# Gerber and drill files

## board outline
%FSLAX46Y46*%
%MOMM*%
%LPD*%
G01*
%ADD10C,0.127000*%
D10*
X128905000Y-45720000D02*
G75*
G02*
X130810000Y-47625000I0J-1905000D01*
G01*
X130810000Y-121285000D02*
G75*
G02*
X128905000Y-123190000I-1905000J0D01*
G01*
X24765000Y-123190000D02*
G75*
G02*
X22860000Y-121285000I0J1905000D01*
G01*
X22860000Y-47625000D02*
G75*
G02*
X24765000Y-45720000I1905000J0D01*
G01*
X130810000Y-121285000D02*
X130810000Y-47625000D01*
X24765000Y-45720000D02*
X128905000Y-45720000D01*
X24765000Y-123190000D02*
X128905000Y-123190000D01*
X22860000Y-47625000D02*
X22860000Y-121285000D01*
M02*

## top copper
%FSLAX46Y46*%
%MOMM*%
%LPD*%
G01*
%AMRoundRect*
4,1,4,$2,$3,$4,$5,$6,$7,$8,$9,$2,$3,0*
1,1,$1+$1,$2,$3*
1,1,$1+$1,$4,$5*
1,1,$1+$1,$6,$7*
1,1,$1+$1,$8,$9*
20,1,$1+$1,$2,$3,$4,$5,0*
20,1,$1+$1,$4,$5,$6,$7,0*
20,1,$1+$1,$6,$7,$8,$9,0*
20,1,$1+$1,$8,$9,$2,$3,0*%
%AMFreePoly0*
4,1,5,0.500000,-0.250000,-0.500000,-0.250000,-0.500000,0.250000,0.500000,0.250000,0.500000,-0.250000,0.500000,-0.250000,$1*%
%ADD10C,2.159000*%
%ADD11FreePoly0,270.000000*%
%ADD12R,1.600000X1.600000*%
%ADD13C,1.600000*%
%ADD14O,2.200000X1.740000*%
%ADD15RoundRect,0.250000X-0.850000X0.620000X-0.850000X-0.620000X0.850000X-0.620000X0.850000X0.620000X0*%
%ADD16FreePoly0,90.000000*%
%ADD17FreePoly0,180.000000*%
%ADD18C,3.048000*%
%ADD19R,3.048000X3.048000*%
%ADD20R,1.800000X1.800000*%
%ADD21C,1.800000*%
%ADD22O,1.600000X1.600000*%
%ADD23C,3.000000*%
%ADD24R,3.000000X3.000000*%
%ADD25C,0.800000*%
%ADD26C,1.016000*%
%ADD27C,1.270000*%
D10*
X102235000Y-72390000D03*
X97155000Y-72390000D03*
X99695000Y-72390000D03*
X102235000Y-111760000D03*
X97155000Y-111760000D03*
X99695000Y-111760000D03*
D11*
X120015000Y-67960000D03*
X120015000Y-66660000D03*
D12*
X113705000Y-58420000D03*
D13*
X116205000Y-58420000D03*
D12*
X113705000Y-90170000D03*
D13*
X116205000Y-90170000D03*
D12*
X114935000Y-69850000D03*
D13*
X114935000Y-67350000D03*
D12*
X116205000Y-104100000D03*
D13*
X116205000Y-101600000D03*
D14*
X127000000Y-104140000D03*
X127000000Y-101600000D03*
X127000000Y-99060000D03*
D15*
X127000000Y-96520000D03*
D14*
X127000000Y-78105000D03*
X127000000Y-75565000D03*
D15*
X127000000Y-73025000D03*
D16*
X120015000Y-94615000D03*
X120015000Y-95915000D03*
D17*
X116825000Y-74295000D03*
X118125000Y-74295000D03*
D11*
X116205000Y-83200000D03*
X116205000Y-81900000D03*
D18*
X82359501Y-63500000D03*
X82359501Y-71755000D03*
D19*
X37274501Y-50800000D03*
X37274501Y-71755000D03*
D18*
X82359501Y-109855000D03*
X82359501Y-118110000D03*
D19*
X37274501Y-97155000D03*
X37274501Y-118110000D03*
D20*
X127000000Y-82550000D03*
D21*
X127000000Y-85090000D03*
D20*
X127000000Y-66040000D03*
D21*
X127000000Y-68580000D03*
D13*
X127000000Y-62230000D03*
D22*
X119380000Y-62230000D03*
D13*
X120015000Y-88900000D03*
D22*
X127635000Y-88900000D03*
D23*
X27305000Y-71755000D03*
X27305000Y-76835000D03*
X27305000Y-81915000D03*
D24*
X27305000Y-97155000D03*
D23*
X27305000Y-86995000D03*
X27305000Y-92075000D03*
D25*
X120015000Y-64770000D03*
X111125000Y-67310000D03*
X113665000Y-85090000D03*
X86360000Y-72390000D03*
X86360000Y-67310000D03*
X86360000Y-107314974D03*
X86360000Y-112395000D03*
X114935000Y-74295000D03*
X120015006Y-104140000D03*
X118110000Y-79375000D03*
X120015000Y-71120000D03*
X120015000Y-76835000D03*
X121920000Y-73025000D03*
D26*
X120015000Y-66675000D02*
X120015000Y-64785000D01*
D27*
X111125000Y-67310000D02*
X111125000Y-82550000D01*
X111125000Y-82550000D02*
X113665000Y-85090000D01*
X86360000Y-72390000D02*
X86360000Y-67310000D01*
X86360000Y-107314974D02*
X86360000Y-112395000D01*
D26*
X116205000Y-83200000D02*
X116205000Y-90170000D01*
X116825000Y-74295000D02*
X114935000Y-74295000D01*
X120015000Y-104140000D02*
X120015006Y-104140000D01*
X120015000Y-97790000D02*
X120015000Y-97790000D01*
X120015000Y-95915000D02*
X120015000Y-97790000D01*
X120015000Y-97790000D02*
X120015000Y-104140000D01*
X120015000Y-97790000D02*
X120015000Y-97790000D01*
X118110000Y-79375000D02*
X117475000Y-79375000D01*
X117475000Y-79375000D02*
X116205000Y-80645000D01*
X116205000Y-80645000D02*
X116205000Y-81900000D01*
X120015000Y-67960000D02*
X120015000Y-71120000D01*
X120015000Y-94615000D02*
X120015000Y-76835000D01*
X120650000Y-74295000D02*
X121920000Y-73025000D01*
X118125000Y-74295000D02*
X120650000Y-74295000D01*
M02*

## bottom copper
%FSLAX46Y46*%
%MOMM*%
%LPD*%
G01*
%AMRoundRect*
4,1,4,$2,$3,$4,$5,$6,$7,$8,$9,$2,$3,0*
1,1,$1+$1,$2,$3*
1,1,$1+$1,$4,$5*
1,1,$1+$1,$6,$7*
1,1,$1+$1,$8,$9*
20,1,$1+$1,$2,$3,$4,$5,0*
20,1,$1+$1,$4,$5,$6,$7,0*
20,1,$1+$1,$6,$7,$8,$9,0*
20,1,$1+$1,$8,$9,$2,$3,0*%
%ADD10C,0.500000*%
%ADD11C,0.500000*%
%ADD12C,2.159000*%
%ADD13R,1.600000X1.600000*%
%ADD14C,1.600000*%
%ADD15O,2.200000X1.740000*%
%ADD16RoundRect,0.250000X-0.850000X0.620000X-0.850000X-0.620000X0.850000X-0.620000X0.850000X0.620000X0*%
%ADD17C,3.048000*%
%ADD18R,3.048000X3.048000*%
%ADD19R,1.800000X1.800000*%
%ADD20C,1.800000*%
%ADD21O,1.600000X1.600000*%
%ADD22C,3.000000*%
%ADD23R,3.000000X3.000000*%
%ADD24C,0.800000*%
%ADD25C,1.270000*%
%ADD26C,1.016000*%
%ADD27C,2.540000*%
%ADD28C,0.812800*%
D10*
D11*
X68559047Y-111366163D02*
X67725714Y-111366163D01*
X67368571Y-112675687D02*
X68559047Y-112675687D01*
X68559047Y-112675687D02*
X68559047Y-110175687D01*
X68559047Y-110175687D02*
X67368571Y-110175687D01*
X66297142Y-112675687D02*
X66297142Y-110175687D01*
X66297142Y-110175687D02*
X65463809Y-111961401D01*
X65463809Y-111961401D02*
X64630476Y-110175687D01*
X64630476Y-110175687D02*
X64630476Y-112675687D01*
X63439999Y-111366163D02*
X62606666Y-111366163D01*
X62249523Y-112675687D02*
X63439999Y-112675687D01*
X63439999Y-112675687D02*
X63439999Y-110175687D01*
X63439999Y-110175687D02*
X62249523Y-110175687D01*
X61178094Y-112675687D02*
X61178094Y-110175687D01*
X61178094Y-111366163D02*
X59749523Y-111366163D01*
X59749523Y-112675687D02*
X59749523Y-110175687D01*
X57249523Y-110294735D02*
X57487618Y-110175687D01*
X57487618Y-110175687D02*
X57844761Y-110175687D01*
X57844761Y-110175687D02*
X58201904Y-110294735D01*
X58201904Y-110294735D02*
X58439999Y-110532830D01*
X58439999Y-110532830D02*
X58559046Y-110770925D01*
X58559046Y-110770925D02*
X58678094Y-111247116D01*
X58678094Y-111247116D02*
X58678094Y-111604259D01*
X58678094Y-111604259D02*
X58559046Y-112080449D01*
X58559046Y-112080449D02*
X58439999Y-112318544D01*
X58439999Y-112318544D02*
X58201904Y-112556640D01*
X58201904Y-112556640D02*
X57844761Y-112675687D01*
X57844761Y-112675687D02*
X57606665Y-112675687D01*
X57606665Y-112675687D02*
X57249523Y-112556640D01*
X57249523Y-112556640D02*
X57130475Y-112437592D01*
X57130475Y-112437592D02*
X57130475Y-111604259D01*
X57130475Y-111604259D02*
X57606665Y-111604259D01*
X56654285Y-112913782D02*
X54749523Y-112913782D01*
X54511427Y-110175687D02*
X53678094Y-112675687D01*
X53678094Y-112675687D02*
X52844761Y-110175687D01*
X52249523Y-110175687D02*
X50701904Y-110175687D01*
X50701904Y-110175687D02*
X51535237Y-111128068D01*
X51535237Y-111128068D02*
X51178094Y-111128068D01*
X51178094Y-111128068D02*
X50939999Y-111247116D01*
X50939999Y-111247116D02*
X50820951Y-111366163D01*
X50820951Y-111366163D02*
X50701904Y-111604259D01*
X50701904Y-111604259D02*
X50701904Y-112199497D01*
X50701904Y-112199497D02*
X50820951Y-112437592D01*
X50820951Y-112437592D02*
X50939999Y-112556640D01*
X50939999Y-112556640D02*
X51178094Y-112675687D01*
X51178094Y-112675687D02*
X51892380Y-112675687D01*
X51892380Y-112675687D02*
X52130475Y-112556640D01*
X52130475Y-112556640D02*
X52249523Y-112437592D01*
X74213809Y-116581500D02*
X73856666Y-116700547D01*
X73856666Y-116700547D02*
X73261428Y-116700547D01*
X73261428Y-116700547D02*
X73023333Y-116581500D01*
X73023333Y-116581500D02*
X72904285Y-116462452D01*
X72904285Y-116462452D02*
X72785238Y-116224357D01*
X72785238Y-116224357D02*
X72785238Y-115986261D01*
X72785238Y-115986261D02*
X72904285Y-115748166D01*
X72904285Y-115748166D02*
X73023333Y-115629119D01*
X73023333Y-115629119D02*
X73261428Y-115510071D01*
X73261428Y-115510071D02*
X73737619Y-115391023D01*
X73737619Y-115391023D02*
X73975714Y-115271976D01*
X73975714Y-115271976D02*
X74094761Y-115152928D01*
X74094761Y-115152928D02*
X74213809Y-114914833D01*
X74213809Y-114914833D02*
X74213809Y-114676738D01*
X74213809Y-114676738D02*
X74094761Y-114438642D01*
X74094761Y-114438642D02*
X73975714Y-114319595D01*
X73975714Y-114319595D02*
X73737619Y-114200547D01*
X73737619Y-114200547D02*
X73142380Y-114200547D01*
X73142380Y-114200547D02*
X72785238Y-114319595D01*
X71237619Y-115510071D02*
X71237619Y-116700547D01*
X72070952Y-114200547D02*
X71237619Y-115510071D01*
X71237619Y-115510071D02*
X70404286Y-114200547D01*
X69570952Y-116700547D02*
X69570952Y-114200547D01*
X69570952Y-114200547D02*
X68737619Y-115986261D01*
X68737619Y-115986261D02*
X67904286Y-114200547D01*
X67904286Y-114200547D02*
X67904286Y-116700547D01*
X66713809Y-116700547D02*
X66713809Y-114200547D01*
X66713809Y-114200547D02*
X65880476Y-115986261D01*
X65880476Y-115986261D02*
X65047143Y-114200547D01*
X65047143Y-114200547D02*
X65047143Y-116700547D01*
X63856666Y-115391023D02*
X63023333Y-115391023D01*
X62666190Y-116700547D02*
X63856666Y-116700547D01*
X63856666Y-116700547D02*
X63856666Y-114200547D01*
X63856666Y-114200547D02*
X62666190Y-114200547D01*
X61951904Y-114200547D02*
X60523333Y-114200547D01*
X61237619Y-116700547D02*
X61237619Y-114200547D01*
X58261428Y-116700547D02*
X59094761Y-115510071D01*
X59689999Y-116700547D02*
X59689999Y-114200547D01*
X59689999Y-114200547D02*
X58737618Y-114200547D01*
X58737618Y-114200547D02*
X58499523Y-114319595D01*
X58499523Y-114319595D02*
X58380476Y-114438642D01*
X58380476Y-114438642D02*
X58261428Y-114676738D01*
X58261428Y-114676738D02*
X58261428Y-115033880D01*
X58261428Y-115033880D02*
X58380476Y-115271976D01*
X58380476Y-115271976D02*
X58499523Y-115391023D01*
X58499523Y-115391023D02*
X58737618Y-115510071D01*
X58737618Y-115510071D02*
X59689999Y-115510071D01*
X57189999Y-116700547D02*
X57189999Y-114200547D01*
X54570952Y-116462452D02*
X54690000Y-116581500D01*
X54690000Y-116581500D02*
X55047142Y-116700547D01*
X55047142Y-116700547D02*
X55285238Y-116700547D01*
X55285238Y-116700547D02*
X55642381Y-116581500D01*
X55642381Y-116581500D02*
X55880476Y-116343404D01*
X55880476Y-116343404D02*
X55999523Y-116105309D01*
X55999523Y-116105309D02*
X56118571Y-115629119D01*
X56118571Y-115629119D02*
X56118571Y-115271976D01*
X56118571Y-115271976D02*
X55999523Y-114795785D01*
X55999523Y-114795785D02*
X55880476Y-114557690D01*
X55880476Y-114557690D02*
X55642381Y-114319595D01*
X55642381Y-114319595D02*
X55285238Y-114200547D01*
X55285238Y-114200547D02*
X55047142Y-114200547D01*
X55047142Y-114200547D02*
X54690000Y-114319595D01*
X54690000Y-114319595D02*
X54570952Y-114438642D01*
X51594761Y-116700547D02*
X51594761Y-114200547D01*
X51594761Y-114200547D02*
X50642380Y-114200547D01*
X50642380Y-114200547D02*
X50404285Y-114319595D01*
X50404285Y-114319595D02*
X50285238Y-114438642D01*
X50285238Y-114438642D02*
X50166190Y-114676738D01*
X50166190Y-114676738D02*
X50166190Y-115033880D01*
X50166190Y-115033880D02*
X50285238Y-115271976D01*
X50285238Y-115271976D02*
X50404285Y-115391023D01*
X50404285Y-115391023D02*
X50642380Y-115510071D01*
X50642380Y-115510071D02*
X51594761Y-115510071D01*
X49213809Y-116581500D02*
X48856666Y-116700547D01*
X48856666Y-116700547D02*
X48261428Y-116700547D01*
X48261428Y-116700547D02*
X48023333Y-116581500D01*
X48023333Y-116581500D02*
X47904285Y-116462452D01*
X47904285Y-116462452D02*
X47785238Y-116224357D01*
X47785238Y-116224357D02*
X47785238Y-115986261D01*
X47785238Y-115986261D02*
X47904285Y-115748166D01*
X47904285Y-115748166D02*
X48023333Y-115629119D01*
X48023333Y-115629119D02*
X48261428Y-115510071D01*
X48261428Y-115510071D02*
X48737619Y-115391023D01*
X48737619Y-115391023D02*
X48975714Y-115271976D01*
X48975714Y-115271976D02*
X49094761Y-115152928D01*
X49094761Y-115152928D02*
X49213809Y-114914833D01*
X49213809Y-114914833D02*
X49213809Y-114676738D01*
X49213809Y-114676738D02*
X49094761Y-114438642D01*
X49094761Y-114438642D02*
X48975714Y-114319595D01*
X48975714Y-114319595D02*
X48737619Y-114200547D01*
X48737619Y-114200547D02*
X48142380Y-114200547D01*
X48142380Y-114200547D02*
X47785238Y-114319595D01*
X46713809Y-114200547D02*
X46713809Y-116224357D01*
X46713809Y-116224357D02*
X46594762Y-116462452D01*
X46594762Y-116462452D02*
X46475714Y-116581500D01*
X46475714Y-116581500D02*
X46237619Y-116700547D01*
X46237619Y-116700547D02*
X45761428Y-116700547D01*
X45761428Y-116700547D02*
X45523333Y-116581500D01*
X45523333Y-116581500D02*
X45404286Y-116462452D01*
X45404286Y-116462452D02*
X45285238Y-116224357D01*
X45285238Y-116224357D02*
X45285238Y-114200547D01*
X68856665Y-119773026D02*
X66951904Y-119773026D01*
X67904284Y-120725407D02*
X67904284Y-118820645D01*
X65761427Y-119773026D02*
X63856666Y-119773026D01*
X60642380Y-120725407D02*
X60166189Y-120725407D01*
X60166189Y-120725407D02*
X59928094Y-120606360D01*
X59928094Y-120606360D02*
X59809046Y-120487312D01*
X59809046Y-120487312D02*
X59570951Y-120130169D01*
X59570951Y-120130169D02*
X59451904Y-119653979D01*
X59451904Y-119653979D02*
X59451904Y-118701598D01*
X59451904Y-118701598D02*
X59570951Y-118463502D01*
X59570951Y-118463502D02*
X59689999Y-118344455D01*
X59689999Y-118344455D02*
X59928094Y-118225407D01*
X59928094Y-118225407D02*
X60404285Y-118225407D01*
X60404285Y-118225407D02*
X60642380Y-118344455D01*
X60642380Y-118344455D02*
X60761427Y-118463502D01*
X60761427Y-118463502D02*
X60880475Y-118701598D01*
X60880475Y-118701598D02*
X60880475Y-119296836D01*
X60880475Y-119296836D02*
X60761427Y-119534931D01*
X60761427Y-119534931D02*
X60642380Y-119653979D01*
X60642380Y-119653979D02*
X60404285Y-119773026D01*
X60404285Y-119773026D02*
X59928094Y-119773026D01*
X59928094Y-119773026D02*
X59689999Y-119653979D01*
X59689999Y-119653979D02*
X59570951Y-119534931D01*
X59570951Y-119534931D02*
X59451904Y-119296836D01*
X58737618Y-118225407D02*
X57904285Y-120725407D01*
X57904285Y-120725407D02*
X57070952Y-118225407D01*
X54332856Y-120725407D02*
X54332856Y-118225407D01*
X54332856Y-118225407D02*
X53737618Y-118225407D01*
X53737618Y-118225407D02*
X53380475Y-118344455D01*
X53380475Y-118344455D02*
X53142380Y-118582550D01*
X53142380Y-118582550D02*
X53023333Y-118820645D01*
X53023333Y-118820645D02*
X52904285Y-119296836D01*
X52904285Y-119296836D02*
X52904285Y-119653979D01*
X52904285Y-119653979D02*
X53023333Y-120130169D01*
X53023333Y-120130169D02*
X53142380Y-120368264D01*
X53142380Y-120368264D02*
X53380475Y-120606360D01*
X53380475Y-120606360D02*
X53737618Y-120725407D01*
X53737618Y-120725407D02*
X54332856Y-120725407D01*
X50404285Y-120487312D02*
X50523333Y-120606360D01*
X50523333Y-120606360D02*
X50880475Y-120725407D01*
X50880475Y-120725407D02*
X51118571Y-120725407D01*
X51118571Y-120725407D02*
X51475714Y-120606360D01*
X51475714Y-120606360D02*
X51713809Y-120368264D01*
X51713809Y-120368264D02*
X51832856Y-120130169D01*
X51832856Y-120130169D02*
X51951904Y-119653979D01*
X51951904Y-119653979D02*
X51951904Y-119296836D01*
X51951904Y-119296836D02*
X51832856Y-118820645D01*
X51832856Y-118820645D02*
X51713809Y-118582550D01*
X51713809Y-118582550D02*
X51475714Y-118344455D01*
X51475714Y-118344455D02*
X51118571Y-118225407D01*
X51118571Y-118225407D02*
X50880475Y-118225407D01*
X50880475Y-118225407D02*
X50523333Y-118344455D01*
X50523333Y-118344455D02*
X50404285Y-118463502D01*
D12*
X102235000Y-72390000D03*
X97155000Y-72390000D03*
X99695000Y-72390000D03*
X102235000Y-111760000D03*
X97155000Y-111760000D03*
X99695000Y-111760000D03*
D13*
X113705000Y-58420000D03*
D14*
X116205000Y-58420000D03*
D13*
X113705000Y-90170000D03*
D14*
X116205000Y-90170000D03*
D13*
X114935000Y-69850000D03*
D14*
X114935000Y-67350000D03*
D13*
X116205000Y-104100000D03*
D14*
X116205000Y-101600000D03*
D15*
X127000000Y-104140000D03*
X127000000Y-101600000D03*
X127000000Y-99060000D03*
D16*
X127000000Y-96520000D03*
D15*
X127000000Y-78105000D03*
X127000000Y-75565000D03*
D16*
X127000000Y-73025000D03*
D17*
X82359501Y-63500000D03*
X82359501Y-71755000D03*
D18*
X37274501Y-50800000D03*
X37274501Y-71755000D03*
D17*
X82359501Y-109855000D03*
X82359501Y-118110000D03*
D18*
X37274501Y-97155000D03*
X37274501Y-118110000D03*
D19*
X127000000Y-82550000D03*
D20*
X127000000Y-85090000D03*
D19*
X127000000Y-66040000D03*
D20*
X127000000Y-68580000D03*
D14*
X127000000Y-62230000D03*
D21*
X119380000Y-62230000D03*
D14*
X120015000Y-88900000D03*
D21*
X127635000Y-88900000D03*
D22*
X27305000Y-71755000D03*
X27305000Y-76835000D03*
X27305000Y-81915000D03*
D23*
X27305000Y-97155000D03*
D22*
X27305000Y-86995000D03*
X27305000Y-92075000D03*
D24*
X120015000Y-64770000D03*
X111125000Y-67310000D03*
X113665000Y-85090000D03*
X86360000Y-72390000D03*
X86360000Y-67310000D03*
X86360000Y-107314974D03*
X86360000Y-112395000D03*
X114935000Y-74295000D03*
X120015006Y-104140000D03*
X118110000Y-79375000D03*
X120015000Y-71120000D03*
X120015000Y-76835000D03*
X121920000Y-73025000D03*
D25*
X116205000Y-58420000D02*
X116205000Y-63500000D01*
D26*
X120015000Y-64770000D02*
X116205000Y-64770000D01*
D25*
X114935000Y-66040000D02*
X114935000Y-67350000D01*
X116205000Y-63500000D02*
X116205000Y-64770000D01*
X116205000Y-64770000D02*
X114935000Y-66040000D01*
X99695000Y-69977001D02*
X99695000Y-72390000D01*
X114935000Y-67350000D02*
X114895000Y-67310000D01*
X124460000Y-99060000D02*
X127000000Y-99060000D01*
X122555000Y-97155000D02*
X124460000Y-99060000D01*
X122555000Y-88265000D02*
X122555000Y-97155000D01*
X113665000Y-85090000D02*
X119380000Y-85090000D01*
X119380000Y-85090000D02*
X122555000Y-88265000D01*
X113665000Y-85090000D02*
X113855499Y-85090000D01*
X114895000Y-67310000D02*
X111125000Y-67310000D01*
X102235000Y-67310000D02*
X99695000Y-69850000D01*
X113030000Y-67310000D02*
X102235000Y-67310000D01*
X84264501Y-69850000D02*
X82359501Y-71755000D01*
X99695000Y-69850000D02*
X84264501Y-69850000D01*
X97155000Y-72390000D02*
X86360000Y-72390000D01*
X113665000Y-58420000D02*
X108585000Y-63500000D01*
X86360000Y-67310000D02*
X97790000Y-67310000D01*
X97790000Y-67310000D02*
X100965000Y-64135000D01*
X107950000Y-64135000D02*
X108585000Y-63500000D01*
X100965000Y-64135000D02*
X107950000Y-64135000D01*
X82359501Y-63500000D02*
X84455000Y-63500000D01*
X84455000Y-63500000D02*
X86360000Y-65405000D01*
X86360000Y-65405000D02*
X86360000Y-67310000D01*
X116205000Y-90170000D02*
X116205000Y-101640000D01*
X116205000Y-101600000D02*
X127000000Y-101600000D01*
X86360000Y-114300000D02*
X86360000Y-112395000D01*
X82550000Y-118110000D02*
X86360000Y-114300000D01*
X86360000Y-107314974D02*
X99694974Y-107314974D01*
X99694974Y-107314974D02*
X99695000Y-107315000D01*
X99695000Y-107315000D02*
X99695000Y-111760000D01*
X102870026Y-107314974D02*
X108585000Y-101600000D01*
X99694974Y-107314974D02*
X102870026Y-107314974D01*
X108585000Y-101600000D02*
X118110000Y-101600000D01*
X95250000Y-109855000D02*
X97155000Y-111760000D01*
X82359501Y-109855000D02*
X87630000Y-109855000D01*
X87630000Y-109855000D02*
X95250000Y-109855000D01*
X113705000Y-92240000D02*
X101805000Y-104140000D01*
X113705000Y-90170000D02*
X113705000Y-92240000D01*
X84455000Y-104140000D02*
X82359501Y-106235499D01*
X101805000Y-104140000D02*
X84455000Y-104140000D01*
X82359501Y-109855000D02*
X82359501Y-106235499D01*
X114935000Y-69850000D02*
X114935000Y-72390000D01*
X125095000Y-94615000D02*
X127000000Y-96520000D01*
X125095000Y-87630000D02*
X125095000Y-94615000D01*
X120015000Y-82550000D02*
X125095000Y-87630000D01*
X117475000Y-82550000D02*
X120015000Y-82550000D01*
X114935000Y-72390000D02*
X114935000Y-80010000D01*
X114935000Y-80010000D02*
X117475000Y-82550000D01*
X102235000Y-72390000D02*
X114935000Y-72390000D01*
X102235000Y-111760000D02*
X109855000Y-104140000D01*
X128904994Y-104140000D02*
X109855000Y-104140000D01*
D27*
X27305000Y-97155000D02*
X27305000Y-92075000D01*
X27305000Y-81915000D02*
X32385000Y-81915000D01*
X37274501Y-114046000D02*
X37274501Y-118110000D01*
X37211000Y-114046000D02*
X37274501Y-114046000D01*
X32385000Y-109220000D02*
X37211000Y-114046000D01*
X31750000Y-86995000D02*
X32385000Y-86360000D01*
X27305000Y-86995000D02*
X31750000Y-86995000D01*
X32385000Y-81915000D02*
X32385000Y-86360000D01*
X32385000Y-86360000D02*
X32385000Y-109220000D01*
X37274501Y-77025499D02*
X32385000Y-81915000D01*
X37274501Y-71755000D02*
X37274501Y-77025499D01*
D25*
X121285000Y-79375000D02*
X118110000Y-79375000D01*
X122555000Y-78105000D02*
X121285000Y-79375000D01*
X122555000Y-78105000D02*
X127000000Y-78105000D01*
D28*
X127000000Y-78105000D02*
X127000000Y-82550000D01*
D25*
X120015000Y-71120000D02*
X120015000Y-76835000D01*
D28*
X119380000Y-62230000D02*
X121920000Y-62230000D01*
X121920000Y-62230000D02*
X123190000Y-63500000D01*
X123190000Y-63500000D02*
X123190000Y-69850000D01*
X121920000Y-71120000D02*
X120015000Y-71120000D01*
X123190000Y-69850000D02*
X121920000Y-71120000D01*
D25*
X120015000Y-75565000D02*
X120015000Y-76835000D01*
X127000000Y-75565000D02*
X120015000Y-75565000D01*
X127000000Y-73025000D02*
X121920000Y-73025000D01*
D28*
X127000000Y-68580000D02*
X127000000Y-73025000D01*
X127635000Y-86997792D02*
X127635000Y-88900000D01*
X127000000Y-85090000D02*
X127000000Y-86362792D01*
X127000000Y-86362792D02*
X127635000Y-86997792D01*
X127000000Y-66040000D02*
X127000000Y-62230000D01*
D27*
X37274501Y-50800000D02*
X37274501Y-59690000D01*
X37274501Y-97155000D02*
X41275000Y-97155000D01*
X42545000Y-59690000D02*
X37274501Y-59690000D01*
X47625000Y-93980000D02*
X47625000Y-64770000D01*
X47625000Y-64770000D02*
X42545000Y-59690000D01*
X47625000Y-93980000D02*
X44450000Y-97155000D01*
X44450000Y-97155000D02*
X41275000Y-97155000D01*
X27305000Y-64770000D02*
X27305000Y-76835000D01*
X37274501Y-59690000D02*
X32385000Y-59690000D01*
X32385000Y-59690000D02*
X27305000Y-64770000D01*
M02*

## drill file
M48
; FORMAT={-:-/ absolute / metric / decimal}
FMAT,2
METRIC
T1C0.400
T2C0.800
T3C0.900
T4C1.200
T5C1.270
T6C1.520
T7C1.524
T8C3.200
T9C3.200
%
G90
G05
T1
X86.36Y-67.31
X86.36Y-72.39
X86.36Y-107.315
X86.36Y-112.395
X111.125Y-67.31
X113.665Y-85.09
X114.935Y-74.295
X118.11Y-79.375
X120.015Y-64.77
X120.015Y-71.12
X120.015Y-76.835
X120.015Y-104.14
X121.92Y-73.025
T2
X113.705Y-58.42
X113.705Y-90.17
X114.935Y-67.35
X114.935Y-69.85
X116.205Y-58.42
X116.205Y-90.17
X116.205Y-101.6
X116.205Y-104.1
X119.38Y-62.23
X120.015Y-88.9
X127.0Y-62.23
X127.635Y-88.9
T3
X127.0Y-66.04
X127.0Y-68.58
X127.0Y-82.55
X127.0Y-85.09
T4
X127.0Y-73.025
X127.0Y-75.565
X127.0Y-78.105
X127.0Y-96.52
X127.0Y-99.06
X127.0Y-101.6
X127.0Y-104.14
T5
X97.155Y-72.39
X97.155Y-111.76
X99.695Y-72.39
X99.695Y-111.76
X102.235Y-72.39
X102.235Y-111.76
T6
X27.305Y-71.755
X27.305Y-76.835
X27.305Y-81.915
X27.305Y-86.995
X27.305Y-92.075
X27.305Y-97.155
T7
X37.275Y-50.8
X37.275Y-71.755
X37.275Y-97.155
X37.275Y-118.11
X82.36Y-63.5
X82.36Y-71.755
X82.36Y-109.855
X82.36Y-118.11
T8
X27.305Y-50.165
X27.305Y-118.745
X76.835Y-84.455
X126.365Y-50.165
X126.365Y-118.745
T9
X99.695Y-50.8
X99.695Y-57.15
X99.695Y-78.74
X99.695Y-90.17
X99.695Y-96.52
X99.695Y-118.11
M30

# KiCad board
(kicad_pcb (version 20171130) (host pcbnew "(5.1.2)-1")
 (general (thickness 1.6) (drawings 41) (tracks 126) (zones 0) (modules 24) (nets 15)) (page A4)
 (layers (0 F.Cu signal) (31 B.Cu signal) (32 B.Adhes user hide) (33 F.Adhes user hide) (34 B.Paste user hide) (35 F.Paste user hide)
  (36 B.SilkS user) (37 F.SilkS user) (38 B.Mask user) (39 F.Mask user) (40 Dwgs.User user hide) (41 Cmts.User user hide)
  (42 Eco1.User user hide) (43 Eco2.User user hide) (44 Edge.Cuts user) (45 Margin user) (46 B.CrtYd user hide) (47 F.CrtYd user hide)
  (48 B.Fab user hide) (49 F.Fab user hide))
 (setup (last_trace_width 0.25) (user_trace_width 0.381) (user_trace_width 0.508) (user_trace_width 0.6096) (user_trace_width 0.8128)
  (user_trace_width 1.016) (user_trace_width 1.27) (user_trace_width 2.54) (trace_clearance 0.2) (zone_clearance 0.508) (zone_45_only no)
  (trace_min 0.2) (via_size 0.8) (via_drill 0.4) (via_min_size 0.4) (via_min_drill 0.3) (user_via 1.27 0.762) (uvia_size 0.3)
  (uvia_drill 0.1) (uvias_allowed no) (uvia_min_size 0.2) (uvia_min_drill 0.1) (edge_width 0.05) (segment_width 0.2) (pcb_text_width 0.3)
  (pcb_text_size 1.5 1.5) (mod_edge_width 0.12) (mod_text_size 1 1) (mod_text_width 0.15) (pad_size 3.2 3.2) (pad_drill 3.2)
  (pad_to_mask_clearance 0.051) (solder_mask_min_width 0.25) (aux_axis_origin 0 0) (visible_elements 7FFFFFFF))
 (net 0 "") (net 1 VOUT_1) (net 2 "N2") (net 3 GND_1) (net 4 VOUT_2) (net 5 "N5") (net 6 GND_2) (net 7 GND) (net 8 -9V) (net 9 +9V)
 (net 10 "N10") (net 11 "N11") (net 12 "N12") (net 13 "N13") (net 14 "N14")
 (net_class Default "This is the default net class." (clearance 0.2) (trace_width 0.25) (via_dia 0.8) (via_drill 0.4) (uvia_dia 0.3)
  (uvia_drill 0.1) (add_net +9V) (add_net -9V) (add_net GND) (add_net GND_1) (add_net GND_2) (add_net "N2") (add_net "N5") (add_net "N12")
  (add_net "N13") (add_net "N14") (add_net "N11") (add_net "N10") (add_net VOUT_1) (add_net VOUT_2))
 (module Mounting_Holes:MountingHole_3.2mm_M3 (layer F.Cu) (at 76.835 84.455)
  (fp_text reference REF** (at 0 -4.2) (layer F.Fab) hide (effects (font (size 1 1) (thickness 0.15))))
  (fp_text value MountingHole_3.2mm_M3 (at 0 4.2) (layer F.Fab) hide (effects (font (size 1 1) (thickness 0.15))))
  (pad "" np_thru_hole circle (at 0 0) (size 3.2 3.2) (drill 3.2) (layers *.Cu *.Mask)))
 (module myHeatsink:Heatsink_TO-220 (layer F.Cu) (at 111.125 82.55 90)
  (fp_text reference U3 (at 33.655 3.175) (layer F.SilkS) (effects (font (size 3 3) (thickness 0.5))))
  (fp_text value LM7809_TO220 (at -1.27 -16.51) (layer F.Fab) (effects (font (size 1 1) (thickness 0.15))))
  (pad "" np_thru_hole circle (at 25.4 -11.43 90) (size 3.2004 3.2004) (drill 3.2004) (layers *.Cu *.Mask))
  (pad 3 thru_hole circle (at 10.16 -8.89 90) (size 2.159 2.159) (drill 1.27) (layers *.Cu *.Mask) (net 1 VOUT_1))
  (pad 1 thru_hole circle (at 10.16 -13.97 90) (size 2.159 2.159) (drill 1.27) (layers *.Cu *.Mask) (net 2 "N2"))
  (pad 2 thru_hole circle (at 10.16 -11.43 90) (size 2.159 2.159) (drill 1.27) (layers *.Cu *.Mask) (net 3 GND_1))
  (pad "" np_thru_hole circle (at 31.75 -11.43 90) (size 3.2004 3.2004) (drill 3.2004) (layers *.Cu *.Mask))
  (pad "" np_thru_hole circle (at 3.81 -11.43 90) (size 3.2004 3.2004) (drill 3.2004) (layers *.Cu *.Mask)))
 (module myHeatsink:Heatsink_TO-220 (layer F.Cu) (at 111.125 121.92 90)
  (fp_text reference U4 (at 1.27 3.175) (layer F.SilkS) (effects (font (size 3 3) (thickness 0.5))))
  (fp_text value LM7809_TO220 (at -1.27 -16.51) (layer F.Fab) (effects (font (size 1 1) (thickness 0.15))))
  (pad "" np_thru_hole circle (at 25.4 -11.43 90) (size 3.2004 3.2004) (drill 3.2004) (layers *.Cu *.Mask))
  (pad 3 thru_hole circle (at 10.16 -8.89 90) (size 2.159 2.159) (drill 1.27) (layers *.Cu *.Mask) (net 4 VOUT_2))
  (pad 1 thru_hole circle (at 10.16 -13.97 90) (size 2.159 2.159) (drill 1.27) (layers *.Cu *.Mask) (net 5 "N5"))
  (pad 2 thru_hole circle (at 10.16 -11.43 90) (size 2.159 2.159) (drill 1.27) (layers *.Cu *.Mask) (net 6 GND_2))
  (pad "" np_thru_hole circle (at 31.75 -11.43 90) (size 3.2004 3.2004) (drill 3.2004) (layers *.Cu *.Mask))
  (pad "" np_thru_hole circle (at 3.81 -11.43 90) (size 3.2004 3.2004) (drill 3.2004) (layers *.Cu *.Mask)))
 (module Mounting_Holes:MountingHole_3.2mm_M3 (layer F.Cu) (at 126.365 118.745)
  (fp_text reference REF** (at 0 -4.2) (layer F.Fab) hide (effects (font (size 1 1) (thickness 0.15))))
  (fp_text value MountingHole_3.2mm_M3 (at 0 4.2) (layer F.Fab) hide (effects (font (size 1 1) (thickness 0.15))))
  (pad 1 np_thru_hole circle (at 0 0) (size 3.2 3.2) (drill 3.2) (layers *.Cu *.Mask)))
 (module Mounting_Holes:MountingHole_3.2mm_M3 (layer F.Cu) (at 126.365 50.165)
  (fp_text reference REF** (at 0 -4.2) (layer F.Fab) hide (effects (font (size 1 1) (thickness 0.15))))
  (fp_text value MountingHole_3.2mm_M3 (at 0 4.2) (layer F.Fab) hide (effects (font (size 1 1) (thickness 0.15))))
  (pad 1 np_thru_hole circle (at 0 0) (size 3.2 3.2) (drill 3.2) (layers *.Cu *.Mask)))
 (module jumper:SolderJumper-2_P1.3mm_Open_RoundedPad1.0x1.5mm (layer F.Cu) (at 120.015 67.31 270)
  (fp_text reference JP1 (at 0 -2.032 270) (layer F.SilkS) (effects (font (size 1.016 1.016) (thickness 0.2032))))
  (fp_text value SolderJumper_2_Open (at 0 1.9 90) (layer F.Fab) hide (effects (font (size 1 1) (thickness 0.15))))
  (pad 2 smd custom (at 0.65 0 270) (size 1 0.5) (layers F.Cu F.Mask) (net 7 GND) (zone_connect 2)
   (options (clearance outline) (anchor rect)) (primitives))
  (pad 1 smd custom (at -0.65 0 270) (size 1 0.5) (layers F.Cu F.Mask) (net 3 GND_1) (zone_connect 2)
   (options (clearance outline) (anchor rect)) (primitives)))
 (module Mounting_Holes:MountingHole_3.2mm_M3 (layer F.Cu) (at 27.305 118.745)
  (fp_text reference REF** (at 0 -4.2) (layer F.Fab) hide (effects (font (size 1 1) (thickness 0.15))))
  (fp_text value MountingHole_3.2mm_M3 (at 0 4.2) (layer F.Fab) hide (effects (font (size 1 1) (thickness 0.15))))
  (pad 1 np_thru_hole circle (at 0 0) (size 3.2 3.2) (drill 3.2) (layers *.Cu *.Mask)))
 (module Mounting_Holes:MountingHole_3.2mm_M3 (layer F.Cu) (at 27.305 50.165)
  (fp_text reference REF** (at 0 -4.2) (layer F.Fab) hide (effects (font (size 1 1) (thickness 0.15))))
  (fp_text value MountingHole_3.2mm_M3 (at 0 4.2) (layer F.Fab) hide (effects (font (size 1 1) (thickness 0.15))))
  (pad 1 np_thru_hole circle (at 0 0) (size 3.2 3.2) (drill 3.2) (layers *.Cu *.Mask)))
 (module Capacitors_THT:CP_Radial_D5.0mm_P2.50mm (layer F.Cu) (at 113.705 58.42)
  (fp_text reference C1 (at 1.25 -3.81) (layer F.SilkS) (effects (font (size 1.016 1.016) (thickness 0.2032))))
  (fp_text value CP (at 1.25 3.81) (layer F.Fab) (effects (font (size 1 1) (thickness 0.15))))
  (pad 1 thru_hole rect (at 0 0) (size 1.6 1.6) (drill 0.8) (layers *.Cu *.Mask) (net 2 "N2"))
  (pad 2 thru_hole circle (at 2.5 0) (size 1.6 1.6) (drill 0.8) (layers *.Cu *.Mask) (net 3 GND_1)))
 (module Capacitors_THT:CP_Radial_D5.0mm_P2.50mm (layer F.Cu) (at 113.705 90.17)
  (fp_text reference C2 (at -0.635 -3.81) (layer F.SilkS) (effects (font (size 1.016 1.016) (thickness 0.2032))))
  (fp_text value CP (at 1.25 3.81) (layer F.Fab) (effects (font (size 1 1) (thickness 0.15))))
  (pad 1 thru_hole rect (at 0 0) (size 1.6 1.6) (drill 0.8) (layers *.Cu *.Mask) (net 5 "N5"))
  (pad 2 thru_hole circle (at 2.5 0) (size 1.6 1.6) (drill 0.8) (layers *.Cu *.Mask) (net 6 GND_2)))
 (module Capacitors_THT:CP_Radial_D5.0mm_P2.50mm (layer F.Cu) (at 114.935 69.85 90)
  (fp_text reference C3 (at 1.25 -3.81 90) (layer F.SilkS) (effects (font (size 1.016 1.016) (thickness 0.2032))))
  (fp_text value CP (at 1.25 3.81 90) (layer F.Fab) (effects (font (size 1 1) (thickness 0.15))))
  (pad 1 thru_hole rect (at 0 0 90) (size 1.6 1.6) (drill 0.8) (layers *.Cu *.Mask) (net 1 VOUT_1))
  (pad 2 thru_hole circle (at 2.5 0 90) (size 1.6 1.6) (drill 0.8) (layers *.Cu *.Mask) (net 3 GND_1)))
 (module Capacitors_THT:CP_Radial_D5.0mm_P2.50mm (layer F.Cu) (at 116.205 104.1 90)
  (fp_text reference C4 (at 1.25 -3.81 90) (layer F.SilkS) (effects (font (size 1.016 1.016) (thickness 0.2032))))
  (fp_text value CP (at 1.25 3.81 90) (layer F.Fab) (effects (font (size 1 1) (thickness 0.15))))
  (pad 1 thru_hole rect (at 0 0 90) (size 1.6 1.6) (drill 0.8) (layers *.Cu *.Mask) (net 4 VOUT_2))
  (pad 2 thru_hole circle (at 2.5 0 90) (size 1.6 1.6) (drill 0.8) (layers *.Cu *.Mask) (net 6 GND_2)))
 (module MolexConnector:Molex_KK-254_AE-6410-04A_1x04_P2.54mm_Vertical (layer F.Cu) (at 127 96.52 270)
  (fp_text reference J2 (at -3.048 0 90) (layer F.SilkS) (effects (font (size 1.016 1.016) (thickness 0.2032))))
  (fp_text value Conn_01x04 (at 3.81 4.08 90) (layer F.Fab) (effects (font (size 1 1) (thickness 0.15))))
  (pad 4 thru_hole oval (at 7.62 0 270) (size 1.74 2.2) (drill 1.2) (layers *.Cu *.Mask) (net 4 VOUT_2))
  (pad 3 thru_hole oval (at 5.08 0 270) (size 1.74 2.2) (drill 1.2) (layers *.Cu *.Mask) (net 6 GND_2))
  (pad 2 thru_hole oval (at 2.54 0 270) (size 1.74 2.2) (drill 1.2) (layers *.Cu *.Mask) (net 3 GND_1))
  (pad 1 thru_hole roundrect (at 0 0 270) (size 1.74 2.2) (drill 1.2) (layers *.Cu *.Mask) (roundrect_rratio 0.143678) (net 1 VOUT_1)))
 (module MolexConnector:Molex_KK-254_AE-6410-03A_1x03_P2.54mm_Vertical (layer F.Cu) (at 127 73.025 270)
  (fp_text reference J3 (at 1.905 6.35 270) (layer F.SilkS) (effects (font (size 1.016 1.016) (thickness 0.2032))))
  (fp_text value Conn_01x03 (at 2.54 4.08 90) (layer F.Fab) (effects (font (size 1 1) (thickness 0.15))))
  (pad 3 thru_hole oval (at 5.08 0 270) (size 1.74 2.2) (drill 1.2) (layers *.Cu *.Mask) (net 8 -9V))
  (pad 2 thru_hole oval (at 2.54 0 270) (size 1.74 2.2) (drill 1.2) (layers *.Cu *.Mask) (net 7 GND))
  (pad 1 thru_hole roundrect (at 0 0 270) (size 1.74 2.2) (drill 1.2) (layers *.Cu *.Mask) (roundrect_rratio 0.143678) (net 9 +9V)))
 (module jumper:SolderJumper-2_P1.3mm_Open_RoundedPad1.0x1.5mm (layer F.Cu) (at 120.015 95.265 90)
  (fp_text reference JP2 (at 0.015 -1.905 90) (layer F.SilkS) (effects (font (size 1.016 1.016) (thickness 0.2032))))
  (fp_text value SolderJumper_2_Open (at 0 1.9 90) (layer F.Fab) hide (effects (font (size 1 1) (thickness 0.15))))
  (pad 2 smd custom (at 0.65 0 90) (size 1 0.5) (layers F.Cu F.Mask) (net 7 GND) (zone_connect 2)
   (options (clearance outline) (anchor rect)) (primitives))
  (pad 1 smd custom (at -0.65 0 90) (size 1 0.5) (layers F.Cu F.Mask) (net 4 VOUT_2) (zone_connect 2)
   (options (clearance outline) (anchor rect)) (primitives)))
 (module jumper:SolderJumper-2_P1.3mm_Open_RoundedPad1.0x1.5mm (layer F.Cu) (at 117.475 74.295 180)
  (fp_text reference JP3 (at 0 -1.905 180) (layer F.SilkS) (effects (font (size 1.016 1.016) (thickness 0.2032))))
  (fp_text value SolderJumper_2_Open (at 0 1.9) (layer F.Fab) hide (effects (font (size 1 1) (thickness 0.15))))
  (pad 2 smd custom (at 0.65 0 180) (size 1 0.5) (layers F.Cu F.Mask) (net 1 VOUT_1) (zone_connect 2)
   (options (clearance outline) (anchor rect)) (primitives))
  (pad 1 smd custom (at -0.65 0 180) (size 1 0.5) (layers F.Cu F.Mask) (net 9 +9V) (zone_connect 2)
   (options (clearance outline) (anchor rect)) (primitives)))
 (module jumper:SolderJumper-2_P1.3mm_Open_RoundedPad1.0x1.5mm (layer F.Cu) (at 116.205 82.55 270)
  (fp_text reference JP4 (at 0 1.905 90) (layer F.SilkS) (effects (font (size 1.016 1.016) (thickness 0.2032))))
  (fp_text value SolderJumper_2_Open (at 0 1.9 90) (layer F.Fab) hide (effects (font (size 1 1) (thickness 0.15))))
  (pad 2 smd custom (at 0.65 0 270) (size 1 0.5) (layers F.Cu F.Mask) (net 6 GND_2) (zone_connect 2)
   (options (clearance outline) (anchor rect)) (primitives))
  (pad 1 smd custom (at -0.65 0 270) (size 1 0.5) (layers F.Cu F.Mask) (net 8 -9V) (zone_connect 2)
   (options (clearance outline) (anchor rect)) (primitives)))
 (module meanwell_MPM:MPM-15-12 (layer F.Cu) (at 37.592001 71.4375)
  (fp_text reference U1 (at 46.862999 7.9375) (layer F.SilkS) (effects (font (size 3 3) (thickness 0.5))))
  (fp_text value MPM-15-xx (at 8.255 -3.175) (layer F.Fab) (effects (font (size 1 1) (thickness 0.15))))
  (pad 4 thru_hole circle (at 44.7675 -7.9375) (size 3.048 3.048) (drill 1.524) (layers *.Cu *.Mask) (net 2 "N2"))
  (pad 3 thru_hole circle (at 44.7675 0.3175) (size 3.048 3.048) (drill 1.524) (layers *.Cu *.Mask) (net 3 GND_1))
  (pad 2 thru_hole rect (at -0.3175 -20.6375) (size 3.048 3.048) (drill 1.524) (layers *.Cu *.Mask) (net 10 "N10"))
  (pad 1 thru_hole rect (at -0.3175 0.3175) (size 3.048 3.048) (drill 1.524) (layers *.Cu *.Mask) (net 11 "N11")))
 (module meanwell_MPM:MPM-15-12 (layer F.Cu) (at 37.592001 117.7925)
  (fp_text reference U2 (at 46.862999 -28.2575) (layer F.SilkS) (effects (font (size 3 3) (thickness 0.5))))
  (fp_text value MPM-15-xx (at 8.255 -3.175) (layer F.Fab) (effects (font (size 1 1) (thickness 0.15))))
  (pad 4 thru_hole circle (at 44.7675 -7.9375) (size 3.048 3.048) (drill 1.524) (layers *.Cu *.Mask) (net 5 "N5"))
  (pad 3 thru_hole circle (at 44.7675 0.3175) (size 3.048 3.048) (drill 1.524) (layers *.Cu *.Mask) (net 6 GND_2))
  (pad 2 thru_hole rect (at -0.3175 -20.6375) (size 3.048 3.048) (drill 1.524) (layers *.Cu *.Mask) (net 10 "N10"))
  (pad 1 thru_hole rect (at -0.3175 0.3175) (size 3.048 3.048) (drill 1.524) (layers *.Cu *.Mask) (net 11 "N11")))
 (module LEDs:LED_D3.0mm (layer F.Cu) (at 127 82.55 270)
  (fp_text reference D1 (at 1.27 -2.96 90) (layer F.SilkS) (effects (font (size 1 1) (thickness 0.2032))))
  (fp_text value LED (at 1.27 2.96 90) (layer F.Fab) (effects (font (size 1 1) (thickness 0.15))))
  (pad 1 thru_hole rect (at 0 0 270) (size 1.8 1.8) (drill 0.9) (layers *.Cu *.Mask) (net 8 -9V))
  (pad 2 thru_hole circle (at 2.54 0 270) (size 1.8 1.8) (drill 0.9) (layers *.Cu *.Mask) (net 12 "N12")))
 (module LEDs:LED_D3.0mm (layer F.Cu) (at 127 66.04 270)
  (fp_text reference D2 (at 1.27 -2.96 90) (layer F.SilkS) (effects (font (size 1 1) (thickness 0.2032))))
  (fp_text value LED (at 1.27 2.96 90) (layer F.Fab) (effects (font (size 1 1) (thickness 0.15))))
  (pad 1 thru_hole rect (at 0 0 270) (size 1.8 1.8) (drill 0.9) (layers *.Cu *.Mask) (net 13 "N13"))
  (pad 2 thru_hole circle (at 2.54 0 270) (size 1.8 1.8) (drill 0.9) (layers *.Cu *.Mask) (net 9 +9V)))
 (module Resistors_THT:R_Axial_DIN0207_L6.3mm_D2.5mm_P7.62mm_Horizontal (layer F.Cu) (at 127 62.23 180)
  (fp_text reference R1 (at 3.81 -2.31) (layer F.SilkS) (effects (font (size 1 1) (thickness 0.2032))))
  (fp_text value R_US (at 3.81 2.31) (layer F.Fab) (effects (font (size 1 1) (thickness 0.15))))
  (pad 1 thru_hole circle (at 0 0 180) (size 1.6 1.6) (drill 0.8) (layers *.Cu *.Mask) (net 13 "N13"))
  (pad 2 thru_hole oval (at 7.62 0 180) (size 1.6 1.6) (drill 0.8) (layers *.Cu *.Mask) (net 7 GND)))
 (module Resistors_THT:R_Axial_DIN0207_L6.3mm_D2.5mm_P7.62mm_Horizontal (layer F.Cu) (at 120.015 88.9)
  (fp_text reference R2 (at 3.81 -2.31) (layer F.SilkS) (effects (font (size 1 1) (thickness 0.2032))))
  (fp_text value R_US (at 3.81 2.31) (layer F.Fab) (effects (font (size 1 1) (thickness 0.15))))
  (pad 1 thru_hole circle (at 0 0) (size 1.6 1.6) (drill 0.8) (layers *.Cu *.Mask) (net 7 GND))
  (pad 2 thru_hole oval (at 7.62 0) (size 1.6 1.6) (drill 0.8) (layers *.Cu *.Mask) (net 12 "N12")))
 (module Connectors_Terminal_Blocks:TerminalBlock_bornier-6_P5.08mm (layer F.Cu) (at 27.305 97.155 90)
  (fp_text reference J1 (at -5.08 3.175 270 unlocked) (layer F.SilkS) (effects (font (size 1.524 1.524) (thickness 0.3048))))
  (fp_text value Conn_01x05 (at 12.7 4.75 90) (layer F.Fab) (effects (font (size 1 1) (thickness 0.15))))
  (pad 6 thru_hole circle (at 25.4 0 90) (size 3 3) (drill 1.52) (layers *.Cu *.Mask) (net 10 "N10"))
  (pad 5 thru_hole circle (at 20.32 0 90) (size 3 3) (drill 1.52) (layers *.Cu *.Mask) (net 10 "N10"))
  (pad 4 thru_hole circle (at 15.24 0 90) (size 3 3) (drill 1.52) (layers *.Cu *.Mask) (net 11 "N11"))
  (pad 1 thru_hole rect (at 0 0 90) (size 3 3) (drill 1.52) (layers *.Cu *.Mask) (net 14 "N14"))
  (pad 3 thru_hole circle (at 10.16 0 90) (size 3 3) (drill 1.52) (layers *.Cu *.Mask) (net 11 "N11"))
  (pad 2 thru_hole circle (at 5.08 0 90) (size 3 3) (drill 1.52) (layers *.Cu *.Mask) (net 14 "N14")))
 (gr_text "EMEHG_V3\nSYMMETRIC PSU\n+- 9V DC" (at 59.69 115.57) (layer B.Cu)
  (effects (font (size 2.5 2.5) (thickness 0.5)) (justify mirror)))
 (gr_arc (start 128.905 47.625) (end 130.81 47.625) (angle -90) (layer Edge.Cuts) (width 0.127))
 (gr_arc (start 128.905 121.285) (end 128.905 123.19) (angle -90) (layer Edge.Cuts) (width 0.127))
 (gr_arc (start 24.765 121.285) (end 22.86 121.285) (angle -90) (layer Edge.Cuts) (width 0.127))
 (gr_arc (start 24.765 47.625) (end 24.765 45.72) (angle -90) (layer Edge.Cuts) (width 0.127))
 (gr_line (start 130.81 121.285) (end 130.81 47.625) (layer Edge.Cuts) (width 0.127))
 (gr_line (start 24.765 45.72) (end 128.905 45.72) (layer Edge.Cuts) (width 0.127))
 (gr_line (start 24.765 123.19) (end 128.905 123.19) (layer Edge.Cuts) (width 0.127))
 (gr_line (start 22.86 47.625) (end 22.86 121.285) (layer Edge.Cuts) (width 0.127))
 (segment (start 116.205 58.42) (end 116.205 63.5) (width 1.27) (layer B.Cu) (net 3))
 (via (at 120.015 64.77) (size 0.8) (drill 0.4) (layers F.Cu B.Cu) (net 3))
 (segment (start 120.015 64.77) (end 116.205 64.77) (width 1.016) (layer B.Cu) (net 3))
 (segment (start 120.015 66.675) (end 120.015 64.785) (width 1.016) (layer F.Cu) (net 3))
 (segment (start 114.935 66.04) (end 114.935 67.35) (width 1.27) (layer B.Cu) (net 3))
 (segment (start 116.205 63.5) (end 116.205 64.77) (width 1.27) (layer B.Cu) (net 3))
 (segment (start 116.205 64.77) (end 114.935 66.04) (width 1.27) (layer B.Cu) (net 3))
 (segment (start 99.695 69.977001) (end 99.695 72.39) (width 1.27) (layer B.Cu) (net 3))
 (segment (start 114.935 67.35) (end 114.895 67.31) (width 1.27) (layer B.Cu) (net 3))
 (segment (start 124.46 99.06) (end 127 99.06) (width 1.27) (layer B.Cu) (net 3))
 (segment (start 122.555 97.155) (end 124.46 99.06) (width 1.27) (layer B.Cu) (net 3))
 (segment (start 122.555 88.265) (end 122.555 97.155) (width 1.27) (layer B.Cu) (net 3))
 (segment (start 113.665 85.09) (end 119.38 85.09) (width 1.27) (layer B.Cu) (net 3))
 (segment (start 119.38 85.09) (end 122.555 88.265) (width 1.27) (layer B.Cu) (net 3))
 (segment (start 113.665 85.09) (end 113.855499 85.09) (width 1.27) (layer B.Cu) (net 3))
 (via (at 111.125 67.31) (size 0.8) (drill 0.4) (layers F.Cu B.Cu) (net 3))
 (segment (start 114.895 67.31) (end 111.125 67.31) (width 1.27) (layer B.Cu) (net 3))
 (segment (start 111.125 67.31) (end 111.125 82.55) (width 1.27) (layer F.Cu) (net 3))
 (via (at 113.665 85.09) (size 0.8) (drill 0.4) (layers F.Cu B.Cu) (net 3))
 (segment (start 111.125 82.55) (end 113.665 85.09) (width 1.27) (layer F.Cu) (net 3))
 (segment (start 102.235 67.31) (end 99.695 69.85) (width 1.27) (layer B.Cu) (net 3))
 (segment (start 113.03 67.31) (end 102.235 67.31) (width 1.27) (layer B.Cu) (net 3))
 (segment (start 84.264501 69.85) (end 82.359501 71.755) (width 1.27) (layer B.Cu) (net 3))
 (segment (start 99.695 69.85) (end 84.264501 69.85) (width 1.27) (layer B.Cu) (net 3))
 (via (at 86.36 72.39) (size 0.8) (drill 0.4) (layers F.Cu B.Cu) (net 2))
 (segment (start 97.155 72.39) (end 86.36 72.39) (width 1.27) (layer B.Cu) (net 2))
 (segment (start 113.665 58.42) (end 108.585 63.5) (width 1.27) (layer B.Cu) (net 2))
 (via (at 86.36 67.31) (size 0.8) (drill 0.4) (layers F.Cu B.Cu) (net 2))
 (segment (start 86.36 72.39) (end 86.36 67.31) (width 1.27) (layer F.Cu) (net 2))
 (segment (start 86.36 67.31) (end 97.79 67.31) (width 1.27) (layer B.Cu) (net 2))
 (segment (start 97.79 67.31) (end 100.965 64.135) (width 1.27) (layer B.Cu) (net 2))
 (segment (start 107.95 64.135) (end 108.585 63.5) (width 1.27) (layer B.Cu) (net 2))
 (segment (start 100.965 64.135) (end 107.95 64.135) (width 1.27) (layer B.Cu) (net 2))
 (segment (start 82.359501 63.5) (end 84.455 63.5) (width 1.27) (layer B.Cu) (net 2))
 (segment (start 84.455 63.5) (end 86.36 65.405) (width 1.27) (layer B.Cu) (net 2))
 (segment (start 86.36 65.405) (end 86.36 67.31) (width 1.27) (layer B.Cu) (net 2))
 (segment (start 116.205 90.17) (end 116.205 101.64) (width 1.27) (layer B.Cu) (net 6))
 (segment (start 116.205 101.6) (end 127 101.6) (width 1.27) (layer B.Cu) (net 6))
 (via (at 86.36 107.314974) (size 0.8) (drill 0.4) (layers F.Cu B.Cu) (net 6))
 (via (at 86.36 112.395) (size 0.8) (drill 0.4) (layers F.Cu B.Cu) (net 6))
 (segment (start 86.36 107.314974) (end 86.36 112.395) (width 1.27) (layer F.Cu) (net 6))
 (segment (start 86.36 114.3) (end 86.36 112.395) (width 1.27) (layer B.Cu) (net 6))
 (segment (start 82.55 118.11) (end 86.36 114.3) (width 1.27) (layer B.Cu) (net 6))
 (segment (start 86.36 107.314974) (end 99.694974 107.314974) (width 1.27) (layer B.Cu) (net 6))
 (segment (start 99.694974 107.314974) (end 99.695 107.315) (width 1.27) (layer B.Cu) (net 6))
 (segment (start 99.695 107.315) (end 99.695 111.76) (width 1.27) (layer B.Cu) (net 6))
 (segment (start 102.870026 107.314974) (end 108.585 101.6) (width 1.27) (layer B.Cu) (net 6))
 (segment (start 99.694974 107.314974) (end 102.870026 107.314974) (width 1.27) (layer B.Cu) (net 6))
 (segment (start 108.585 101.6) (end 118.11 101.6) (width 1.27) (layer B.Cu) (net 6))
 (segment (start 116.205 83.2) (end 116.205 90.17) (width 1.016) (layer F.Cu) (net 6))
 (segment (start 95.25 109.855) (end 97.155 111.76) (width 1.27) (layer B.Cu) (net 5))
 (segment (start 82.359501 109.855) (end 87.63 109.855) (width 1.27) (layer B.Cu) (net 5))
 (segment (start 87.63 109.855) (end 95.25 109.855) (width 1.27) (layer B.Cu) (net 5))
 (segment (start 113.705 92.24) (end 101.805 104.14) (width 1.27) (layer B.Cu) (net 5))
 (segment (start 113.705 90.17) (end 113.705 92.24) (width 1.27) (layer B.Cu) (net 5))
 (segment (start 84.455 104.14) (end 82.359501 106.235499) (width 1.27) (layer B.Cu) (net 5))
 (segment (start 101.805 104.14) (end 84.455 104.14) (width 1.27) (layer B.Cu) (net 5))
 (segment (start 82.359501 109.855) (end 82.359501 106.235499) (width 1.27) (layer B.Cu) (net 5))
 (segment (start 114.935 69.85) (end 114.935 72.39) (width 1.27) (layer B.Cu) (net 1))
 (via (at 114.935 74.295) (size 0.8) (drill 0.4) (layers F.Cu B.Cu) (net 1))
 (segment (start 116.825 74.295) (end 114.935 74.295) (width 1.016) (layer F.Cu) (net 1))
 (segment (start 125.095 94.615) (end 127 96.52) (width 1.27) (layer B.Cu) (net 1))
 (segment (start 125.095 87.63) (end 125.095 94.615) (width 1.27) (layer B.Cu) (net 1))
 (segment (start 120.015 82.55) (end 125.095 87.63) (width 1.27) (layer B.Cu) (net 1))
 (segment (start 117.475 82.55) (end 120.015 82.55) (width 1.27) (layer B.Cu) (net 1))
 (segment (start 114.935 72.39) (end 114.935 80.01) (width 1.27) (layer B.Cu) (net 1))
 (segment (start 114.935 80.01) (end 117.475 82.55) (width 1.27) (layer B.Cu) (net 1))
 (segment (start 102.235 72.39) (end 114.935 72.39) (width 1.27) (layer B.Cu) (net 1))
 (via (at 120.015006 104.14) (size 0.8) (drill 0.4) (layers F.Cu B.Cu) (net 4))
 (segment (start 120.015 104.14) (end 120.015006 104.14) (width 1.016) (layer F.Cu) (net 4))
 (segment (start 120.015 97.79) (end 120.015 97.79) (width 1.016) (layer F.Cu) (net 4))
 (segment (start 120.015 95.915) (end 120.015 97.79) (width 1.016) (layer F.Cu) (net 4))
 (segment (start 120.015 97.79) (end 120.015 104.14) (width 1.016) (layer F.Cu) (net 4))
 (segment (start 120.015 97.79) (end 120.015 97.79) (width 1.016) (layer F.Cu) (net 4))
 (segment (start 102.235 111.76) (end 109.855 104.14) (width 1.27) (layer B.Cu) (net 4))
 (segment (start 128.904994 104.14) (end 109.855 104.14) (width 1.27) (layer B.Cu) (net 4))
 (segment (start 27.305 97.155) (end 27.305 92.075) (width 2.54) (layer B.Cu) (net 14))
 (segment (start 27.305 81.915) (end 32.385 81.915) (width 2.54) (layer B.Cu) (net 11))
 (segment (start 37.274501 114.046) (end 37.274501 118.11) (width 2.54) (layer B.Cu) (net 11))
 (segment (start 37.211 114.046) (end 37.274501 114.046) (width 2.54) (layer B.Cu) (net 11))
 (segment (start 32.385 109.22) (end 37.211 114.046) (width 2.54) (layer B.Cu) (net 11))
 (segment (start 31.75 86.995) (end 32.385 86.36) (width 2.54) (layer B.Cu) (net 11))
 (segment (start 27.305 86.995) (end 31.75 86.995) (width 2.54) (layer B.Cu) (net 11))
 (segment (start 32.385 81.915) (end 32.385 86.36) (width 2.54) (layer B.Cu) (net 11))
 (segment (start 32.385 86.36) (end 32.385 109.22) (width 2.54) (layer B.Cu) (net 11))
 (segment (start 37.274501 77.025499) (end 32.385 81.915) (width 2.54) (layer B.Cu) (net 11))
 (segment (start 37.274501 71.755) (end 37.274501 77.025499) (width 2.54) (layer B.Cu) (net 11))
 (via (at 118.11 79.375) (size 0.8) (drill 0.4) (layers F.Cu B.Cu) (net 8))
 (segment (start 118.11 79.375) (end 117.475 79.375) (width 1.016) (layer F.Cu) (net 8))
 (segment (start 117.475 79.375) (end 116.205 80.645) (width 1.016) (layer F.Cu) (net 8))
 (segment (start 116.205 80.645) (end 116.205 81.9) (width 1.016) (layer F.Cu) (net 8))
 (segment (start 121.285 79.375) (end 118.11 79.375) (width 1.27) (layer B.Cu) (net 8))
 (segment (start 122.555 78.105) (end 121.285 79.375) (width 1.27) (layer B.Cu) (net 8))
 (segment (start 122.555 78.105) (end 127 78.105) (width 1.27) (layer B.Cu) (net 8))
 (segment (start 127 78.105) (end 127 82.55) (width 0.8128) (layer B.Cu) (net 8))
 (via (at 120.015 71.12) (size 0.8) (drill 0.4) (layers F.Cu B.Cu) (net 7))
 (segment (start 120.015 67.96) (end 120.015 71.12) (width 1.016) (layer F.Cu) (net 7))
 (via (at 120.015 76.835) (size 0.8) (drill 0.4) (layers F.Cu B.Cu) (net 7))
 (segment (start 120.015 94.615) (end 120.015 76.835) (width 1.016) (layer F.Cu) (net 7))
 (segment (start 120.015 71.12) (end 120.015 76.835) (width 1.27) (layer B.Cu) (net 7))
 (segment (start 119.38 62.23) (end 121.92 62.23) (width 0.8128) (layer B.Cu) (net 7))
 (segment (start 121.92 62.23) (end 123.19 63.5) (width 0.8128) (layer B.Cu) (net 7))
 (segment (start 123.19 63.5) (end 123.19 69.85) (width 0.8128) (layer B.Cu) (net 7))
 (segment (start 121.92 71.12) (end 120.015 71.12) (width 0.8128) (layer B.Cu) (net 7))
 (segment (start 123.19 69.85) (end 121.92 71.12) (width 0.8128) (layer B.Cu) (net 7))
 (segment (start 120.015 75.565) (end 120.015 76.835) (width 1.27) (layer B.Cu) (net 7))
 (segment (start 127 75.565) (end 120.015 75.565) (width 1.27) (layer B.Cu) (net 7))
 (via (at 121.92 73.025) (size 0.8) (drill 0.4) (layers F.Cu B.Cu) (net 9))
 (segment (start 127 73.025) (end 121.92 73.025) (width 1.27) (layer B.Cu) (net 9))
 (segment (start 120.65 74.295) (end 121.92 73.025) (width 1.016) (layer F.Cu) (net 9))
 (segment (start 118.125 74.295) (end 120.65 74.295) (width 1.016) (layer F.Cu) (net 9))
 (segment (start 127 68.58) (end 127 73.025) (width 0.8128) (layer B.Cu) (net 9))
 (segment (start 127.635 86.997792) (end 127.635 88.9) (width 0.8128) (layer B.Cu) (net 12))
 (segment (start 127 85.09) (end 127 86.362792) (width 0.8128) (layer B.Cu) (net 12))
 (segment (start 127 86.362792) (end 127.635 86.997792) (width 0.8128) (layer B.Cu) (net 12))
 (segment (start 127 66.04) (end 127 62.23) (width 0.8128) (layer B.Cu) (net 13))
 (segment (start 37.274501 50.8) (end 37.274501 59.69) (width 2.54) (layer B.Cu) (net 10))
 (segment (start 37.274501 97.155) (end 41.275 97.155) (width 2.54) (layer B.Cu) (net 10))
 (segment (start 42.545 59.69) (end 37.274501 59.69) (width 2.54) (layer B.Cu) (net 10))
 (segment (start 47.625 93.98) (end 47.625 64.77) (width 2.54) (layer B.Cu) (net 10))
 (segment (start 47.625 64.77) (end 42.545 59.69) (width 2.54) (layer B.Cu) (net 10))
 (segment (start 47.625 93.98) (end 44.45 97.155) (width 2.54) (layer B.Cu) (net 10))
 (segment (start 44.45 97.155) (end 41.275 97.155) (width 2.54) (layer B.Cu) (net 10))
 (segment (start 27.305 64.77) (end 27.305 76.835) (width 2.54) (layer B.Cu) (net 10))
 (segment (start 37.274501 59.69) (end 32.385 59.69) (width 2.54) (layer B.Cu) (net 10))
 (segment (start 32.385 59.69) (end 27.305 64.77) (width 2.54) (layer B.Cu) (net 10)))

